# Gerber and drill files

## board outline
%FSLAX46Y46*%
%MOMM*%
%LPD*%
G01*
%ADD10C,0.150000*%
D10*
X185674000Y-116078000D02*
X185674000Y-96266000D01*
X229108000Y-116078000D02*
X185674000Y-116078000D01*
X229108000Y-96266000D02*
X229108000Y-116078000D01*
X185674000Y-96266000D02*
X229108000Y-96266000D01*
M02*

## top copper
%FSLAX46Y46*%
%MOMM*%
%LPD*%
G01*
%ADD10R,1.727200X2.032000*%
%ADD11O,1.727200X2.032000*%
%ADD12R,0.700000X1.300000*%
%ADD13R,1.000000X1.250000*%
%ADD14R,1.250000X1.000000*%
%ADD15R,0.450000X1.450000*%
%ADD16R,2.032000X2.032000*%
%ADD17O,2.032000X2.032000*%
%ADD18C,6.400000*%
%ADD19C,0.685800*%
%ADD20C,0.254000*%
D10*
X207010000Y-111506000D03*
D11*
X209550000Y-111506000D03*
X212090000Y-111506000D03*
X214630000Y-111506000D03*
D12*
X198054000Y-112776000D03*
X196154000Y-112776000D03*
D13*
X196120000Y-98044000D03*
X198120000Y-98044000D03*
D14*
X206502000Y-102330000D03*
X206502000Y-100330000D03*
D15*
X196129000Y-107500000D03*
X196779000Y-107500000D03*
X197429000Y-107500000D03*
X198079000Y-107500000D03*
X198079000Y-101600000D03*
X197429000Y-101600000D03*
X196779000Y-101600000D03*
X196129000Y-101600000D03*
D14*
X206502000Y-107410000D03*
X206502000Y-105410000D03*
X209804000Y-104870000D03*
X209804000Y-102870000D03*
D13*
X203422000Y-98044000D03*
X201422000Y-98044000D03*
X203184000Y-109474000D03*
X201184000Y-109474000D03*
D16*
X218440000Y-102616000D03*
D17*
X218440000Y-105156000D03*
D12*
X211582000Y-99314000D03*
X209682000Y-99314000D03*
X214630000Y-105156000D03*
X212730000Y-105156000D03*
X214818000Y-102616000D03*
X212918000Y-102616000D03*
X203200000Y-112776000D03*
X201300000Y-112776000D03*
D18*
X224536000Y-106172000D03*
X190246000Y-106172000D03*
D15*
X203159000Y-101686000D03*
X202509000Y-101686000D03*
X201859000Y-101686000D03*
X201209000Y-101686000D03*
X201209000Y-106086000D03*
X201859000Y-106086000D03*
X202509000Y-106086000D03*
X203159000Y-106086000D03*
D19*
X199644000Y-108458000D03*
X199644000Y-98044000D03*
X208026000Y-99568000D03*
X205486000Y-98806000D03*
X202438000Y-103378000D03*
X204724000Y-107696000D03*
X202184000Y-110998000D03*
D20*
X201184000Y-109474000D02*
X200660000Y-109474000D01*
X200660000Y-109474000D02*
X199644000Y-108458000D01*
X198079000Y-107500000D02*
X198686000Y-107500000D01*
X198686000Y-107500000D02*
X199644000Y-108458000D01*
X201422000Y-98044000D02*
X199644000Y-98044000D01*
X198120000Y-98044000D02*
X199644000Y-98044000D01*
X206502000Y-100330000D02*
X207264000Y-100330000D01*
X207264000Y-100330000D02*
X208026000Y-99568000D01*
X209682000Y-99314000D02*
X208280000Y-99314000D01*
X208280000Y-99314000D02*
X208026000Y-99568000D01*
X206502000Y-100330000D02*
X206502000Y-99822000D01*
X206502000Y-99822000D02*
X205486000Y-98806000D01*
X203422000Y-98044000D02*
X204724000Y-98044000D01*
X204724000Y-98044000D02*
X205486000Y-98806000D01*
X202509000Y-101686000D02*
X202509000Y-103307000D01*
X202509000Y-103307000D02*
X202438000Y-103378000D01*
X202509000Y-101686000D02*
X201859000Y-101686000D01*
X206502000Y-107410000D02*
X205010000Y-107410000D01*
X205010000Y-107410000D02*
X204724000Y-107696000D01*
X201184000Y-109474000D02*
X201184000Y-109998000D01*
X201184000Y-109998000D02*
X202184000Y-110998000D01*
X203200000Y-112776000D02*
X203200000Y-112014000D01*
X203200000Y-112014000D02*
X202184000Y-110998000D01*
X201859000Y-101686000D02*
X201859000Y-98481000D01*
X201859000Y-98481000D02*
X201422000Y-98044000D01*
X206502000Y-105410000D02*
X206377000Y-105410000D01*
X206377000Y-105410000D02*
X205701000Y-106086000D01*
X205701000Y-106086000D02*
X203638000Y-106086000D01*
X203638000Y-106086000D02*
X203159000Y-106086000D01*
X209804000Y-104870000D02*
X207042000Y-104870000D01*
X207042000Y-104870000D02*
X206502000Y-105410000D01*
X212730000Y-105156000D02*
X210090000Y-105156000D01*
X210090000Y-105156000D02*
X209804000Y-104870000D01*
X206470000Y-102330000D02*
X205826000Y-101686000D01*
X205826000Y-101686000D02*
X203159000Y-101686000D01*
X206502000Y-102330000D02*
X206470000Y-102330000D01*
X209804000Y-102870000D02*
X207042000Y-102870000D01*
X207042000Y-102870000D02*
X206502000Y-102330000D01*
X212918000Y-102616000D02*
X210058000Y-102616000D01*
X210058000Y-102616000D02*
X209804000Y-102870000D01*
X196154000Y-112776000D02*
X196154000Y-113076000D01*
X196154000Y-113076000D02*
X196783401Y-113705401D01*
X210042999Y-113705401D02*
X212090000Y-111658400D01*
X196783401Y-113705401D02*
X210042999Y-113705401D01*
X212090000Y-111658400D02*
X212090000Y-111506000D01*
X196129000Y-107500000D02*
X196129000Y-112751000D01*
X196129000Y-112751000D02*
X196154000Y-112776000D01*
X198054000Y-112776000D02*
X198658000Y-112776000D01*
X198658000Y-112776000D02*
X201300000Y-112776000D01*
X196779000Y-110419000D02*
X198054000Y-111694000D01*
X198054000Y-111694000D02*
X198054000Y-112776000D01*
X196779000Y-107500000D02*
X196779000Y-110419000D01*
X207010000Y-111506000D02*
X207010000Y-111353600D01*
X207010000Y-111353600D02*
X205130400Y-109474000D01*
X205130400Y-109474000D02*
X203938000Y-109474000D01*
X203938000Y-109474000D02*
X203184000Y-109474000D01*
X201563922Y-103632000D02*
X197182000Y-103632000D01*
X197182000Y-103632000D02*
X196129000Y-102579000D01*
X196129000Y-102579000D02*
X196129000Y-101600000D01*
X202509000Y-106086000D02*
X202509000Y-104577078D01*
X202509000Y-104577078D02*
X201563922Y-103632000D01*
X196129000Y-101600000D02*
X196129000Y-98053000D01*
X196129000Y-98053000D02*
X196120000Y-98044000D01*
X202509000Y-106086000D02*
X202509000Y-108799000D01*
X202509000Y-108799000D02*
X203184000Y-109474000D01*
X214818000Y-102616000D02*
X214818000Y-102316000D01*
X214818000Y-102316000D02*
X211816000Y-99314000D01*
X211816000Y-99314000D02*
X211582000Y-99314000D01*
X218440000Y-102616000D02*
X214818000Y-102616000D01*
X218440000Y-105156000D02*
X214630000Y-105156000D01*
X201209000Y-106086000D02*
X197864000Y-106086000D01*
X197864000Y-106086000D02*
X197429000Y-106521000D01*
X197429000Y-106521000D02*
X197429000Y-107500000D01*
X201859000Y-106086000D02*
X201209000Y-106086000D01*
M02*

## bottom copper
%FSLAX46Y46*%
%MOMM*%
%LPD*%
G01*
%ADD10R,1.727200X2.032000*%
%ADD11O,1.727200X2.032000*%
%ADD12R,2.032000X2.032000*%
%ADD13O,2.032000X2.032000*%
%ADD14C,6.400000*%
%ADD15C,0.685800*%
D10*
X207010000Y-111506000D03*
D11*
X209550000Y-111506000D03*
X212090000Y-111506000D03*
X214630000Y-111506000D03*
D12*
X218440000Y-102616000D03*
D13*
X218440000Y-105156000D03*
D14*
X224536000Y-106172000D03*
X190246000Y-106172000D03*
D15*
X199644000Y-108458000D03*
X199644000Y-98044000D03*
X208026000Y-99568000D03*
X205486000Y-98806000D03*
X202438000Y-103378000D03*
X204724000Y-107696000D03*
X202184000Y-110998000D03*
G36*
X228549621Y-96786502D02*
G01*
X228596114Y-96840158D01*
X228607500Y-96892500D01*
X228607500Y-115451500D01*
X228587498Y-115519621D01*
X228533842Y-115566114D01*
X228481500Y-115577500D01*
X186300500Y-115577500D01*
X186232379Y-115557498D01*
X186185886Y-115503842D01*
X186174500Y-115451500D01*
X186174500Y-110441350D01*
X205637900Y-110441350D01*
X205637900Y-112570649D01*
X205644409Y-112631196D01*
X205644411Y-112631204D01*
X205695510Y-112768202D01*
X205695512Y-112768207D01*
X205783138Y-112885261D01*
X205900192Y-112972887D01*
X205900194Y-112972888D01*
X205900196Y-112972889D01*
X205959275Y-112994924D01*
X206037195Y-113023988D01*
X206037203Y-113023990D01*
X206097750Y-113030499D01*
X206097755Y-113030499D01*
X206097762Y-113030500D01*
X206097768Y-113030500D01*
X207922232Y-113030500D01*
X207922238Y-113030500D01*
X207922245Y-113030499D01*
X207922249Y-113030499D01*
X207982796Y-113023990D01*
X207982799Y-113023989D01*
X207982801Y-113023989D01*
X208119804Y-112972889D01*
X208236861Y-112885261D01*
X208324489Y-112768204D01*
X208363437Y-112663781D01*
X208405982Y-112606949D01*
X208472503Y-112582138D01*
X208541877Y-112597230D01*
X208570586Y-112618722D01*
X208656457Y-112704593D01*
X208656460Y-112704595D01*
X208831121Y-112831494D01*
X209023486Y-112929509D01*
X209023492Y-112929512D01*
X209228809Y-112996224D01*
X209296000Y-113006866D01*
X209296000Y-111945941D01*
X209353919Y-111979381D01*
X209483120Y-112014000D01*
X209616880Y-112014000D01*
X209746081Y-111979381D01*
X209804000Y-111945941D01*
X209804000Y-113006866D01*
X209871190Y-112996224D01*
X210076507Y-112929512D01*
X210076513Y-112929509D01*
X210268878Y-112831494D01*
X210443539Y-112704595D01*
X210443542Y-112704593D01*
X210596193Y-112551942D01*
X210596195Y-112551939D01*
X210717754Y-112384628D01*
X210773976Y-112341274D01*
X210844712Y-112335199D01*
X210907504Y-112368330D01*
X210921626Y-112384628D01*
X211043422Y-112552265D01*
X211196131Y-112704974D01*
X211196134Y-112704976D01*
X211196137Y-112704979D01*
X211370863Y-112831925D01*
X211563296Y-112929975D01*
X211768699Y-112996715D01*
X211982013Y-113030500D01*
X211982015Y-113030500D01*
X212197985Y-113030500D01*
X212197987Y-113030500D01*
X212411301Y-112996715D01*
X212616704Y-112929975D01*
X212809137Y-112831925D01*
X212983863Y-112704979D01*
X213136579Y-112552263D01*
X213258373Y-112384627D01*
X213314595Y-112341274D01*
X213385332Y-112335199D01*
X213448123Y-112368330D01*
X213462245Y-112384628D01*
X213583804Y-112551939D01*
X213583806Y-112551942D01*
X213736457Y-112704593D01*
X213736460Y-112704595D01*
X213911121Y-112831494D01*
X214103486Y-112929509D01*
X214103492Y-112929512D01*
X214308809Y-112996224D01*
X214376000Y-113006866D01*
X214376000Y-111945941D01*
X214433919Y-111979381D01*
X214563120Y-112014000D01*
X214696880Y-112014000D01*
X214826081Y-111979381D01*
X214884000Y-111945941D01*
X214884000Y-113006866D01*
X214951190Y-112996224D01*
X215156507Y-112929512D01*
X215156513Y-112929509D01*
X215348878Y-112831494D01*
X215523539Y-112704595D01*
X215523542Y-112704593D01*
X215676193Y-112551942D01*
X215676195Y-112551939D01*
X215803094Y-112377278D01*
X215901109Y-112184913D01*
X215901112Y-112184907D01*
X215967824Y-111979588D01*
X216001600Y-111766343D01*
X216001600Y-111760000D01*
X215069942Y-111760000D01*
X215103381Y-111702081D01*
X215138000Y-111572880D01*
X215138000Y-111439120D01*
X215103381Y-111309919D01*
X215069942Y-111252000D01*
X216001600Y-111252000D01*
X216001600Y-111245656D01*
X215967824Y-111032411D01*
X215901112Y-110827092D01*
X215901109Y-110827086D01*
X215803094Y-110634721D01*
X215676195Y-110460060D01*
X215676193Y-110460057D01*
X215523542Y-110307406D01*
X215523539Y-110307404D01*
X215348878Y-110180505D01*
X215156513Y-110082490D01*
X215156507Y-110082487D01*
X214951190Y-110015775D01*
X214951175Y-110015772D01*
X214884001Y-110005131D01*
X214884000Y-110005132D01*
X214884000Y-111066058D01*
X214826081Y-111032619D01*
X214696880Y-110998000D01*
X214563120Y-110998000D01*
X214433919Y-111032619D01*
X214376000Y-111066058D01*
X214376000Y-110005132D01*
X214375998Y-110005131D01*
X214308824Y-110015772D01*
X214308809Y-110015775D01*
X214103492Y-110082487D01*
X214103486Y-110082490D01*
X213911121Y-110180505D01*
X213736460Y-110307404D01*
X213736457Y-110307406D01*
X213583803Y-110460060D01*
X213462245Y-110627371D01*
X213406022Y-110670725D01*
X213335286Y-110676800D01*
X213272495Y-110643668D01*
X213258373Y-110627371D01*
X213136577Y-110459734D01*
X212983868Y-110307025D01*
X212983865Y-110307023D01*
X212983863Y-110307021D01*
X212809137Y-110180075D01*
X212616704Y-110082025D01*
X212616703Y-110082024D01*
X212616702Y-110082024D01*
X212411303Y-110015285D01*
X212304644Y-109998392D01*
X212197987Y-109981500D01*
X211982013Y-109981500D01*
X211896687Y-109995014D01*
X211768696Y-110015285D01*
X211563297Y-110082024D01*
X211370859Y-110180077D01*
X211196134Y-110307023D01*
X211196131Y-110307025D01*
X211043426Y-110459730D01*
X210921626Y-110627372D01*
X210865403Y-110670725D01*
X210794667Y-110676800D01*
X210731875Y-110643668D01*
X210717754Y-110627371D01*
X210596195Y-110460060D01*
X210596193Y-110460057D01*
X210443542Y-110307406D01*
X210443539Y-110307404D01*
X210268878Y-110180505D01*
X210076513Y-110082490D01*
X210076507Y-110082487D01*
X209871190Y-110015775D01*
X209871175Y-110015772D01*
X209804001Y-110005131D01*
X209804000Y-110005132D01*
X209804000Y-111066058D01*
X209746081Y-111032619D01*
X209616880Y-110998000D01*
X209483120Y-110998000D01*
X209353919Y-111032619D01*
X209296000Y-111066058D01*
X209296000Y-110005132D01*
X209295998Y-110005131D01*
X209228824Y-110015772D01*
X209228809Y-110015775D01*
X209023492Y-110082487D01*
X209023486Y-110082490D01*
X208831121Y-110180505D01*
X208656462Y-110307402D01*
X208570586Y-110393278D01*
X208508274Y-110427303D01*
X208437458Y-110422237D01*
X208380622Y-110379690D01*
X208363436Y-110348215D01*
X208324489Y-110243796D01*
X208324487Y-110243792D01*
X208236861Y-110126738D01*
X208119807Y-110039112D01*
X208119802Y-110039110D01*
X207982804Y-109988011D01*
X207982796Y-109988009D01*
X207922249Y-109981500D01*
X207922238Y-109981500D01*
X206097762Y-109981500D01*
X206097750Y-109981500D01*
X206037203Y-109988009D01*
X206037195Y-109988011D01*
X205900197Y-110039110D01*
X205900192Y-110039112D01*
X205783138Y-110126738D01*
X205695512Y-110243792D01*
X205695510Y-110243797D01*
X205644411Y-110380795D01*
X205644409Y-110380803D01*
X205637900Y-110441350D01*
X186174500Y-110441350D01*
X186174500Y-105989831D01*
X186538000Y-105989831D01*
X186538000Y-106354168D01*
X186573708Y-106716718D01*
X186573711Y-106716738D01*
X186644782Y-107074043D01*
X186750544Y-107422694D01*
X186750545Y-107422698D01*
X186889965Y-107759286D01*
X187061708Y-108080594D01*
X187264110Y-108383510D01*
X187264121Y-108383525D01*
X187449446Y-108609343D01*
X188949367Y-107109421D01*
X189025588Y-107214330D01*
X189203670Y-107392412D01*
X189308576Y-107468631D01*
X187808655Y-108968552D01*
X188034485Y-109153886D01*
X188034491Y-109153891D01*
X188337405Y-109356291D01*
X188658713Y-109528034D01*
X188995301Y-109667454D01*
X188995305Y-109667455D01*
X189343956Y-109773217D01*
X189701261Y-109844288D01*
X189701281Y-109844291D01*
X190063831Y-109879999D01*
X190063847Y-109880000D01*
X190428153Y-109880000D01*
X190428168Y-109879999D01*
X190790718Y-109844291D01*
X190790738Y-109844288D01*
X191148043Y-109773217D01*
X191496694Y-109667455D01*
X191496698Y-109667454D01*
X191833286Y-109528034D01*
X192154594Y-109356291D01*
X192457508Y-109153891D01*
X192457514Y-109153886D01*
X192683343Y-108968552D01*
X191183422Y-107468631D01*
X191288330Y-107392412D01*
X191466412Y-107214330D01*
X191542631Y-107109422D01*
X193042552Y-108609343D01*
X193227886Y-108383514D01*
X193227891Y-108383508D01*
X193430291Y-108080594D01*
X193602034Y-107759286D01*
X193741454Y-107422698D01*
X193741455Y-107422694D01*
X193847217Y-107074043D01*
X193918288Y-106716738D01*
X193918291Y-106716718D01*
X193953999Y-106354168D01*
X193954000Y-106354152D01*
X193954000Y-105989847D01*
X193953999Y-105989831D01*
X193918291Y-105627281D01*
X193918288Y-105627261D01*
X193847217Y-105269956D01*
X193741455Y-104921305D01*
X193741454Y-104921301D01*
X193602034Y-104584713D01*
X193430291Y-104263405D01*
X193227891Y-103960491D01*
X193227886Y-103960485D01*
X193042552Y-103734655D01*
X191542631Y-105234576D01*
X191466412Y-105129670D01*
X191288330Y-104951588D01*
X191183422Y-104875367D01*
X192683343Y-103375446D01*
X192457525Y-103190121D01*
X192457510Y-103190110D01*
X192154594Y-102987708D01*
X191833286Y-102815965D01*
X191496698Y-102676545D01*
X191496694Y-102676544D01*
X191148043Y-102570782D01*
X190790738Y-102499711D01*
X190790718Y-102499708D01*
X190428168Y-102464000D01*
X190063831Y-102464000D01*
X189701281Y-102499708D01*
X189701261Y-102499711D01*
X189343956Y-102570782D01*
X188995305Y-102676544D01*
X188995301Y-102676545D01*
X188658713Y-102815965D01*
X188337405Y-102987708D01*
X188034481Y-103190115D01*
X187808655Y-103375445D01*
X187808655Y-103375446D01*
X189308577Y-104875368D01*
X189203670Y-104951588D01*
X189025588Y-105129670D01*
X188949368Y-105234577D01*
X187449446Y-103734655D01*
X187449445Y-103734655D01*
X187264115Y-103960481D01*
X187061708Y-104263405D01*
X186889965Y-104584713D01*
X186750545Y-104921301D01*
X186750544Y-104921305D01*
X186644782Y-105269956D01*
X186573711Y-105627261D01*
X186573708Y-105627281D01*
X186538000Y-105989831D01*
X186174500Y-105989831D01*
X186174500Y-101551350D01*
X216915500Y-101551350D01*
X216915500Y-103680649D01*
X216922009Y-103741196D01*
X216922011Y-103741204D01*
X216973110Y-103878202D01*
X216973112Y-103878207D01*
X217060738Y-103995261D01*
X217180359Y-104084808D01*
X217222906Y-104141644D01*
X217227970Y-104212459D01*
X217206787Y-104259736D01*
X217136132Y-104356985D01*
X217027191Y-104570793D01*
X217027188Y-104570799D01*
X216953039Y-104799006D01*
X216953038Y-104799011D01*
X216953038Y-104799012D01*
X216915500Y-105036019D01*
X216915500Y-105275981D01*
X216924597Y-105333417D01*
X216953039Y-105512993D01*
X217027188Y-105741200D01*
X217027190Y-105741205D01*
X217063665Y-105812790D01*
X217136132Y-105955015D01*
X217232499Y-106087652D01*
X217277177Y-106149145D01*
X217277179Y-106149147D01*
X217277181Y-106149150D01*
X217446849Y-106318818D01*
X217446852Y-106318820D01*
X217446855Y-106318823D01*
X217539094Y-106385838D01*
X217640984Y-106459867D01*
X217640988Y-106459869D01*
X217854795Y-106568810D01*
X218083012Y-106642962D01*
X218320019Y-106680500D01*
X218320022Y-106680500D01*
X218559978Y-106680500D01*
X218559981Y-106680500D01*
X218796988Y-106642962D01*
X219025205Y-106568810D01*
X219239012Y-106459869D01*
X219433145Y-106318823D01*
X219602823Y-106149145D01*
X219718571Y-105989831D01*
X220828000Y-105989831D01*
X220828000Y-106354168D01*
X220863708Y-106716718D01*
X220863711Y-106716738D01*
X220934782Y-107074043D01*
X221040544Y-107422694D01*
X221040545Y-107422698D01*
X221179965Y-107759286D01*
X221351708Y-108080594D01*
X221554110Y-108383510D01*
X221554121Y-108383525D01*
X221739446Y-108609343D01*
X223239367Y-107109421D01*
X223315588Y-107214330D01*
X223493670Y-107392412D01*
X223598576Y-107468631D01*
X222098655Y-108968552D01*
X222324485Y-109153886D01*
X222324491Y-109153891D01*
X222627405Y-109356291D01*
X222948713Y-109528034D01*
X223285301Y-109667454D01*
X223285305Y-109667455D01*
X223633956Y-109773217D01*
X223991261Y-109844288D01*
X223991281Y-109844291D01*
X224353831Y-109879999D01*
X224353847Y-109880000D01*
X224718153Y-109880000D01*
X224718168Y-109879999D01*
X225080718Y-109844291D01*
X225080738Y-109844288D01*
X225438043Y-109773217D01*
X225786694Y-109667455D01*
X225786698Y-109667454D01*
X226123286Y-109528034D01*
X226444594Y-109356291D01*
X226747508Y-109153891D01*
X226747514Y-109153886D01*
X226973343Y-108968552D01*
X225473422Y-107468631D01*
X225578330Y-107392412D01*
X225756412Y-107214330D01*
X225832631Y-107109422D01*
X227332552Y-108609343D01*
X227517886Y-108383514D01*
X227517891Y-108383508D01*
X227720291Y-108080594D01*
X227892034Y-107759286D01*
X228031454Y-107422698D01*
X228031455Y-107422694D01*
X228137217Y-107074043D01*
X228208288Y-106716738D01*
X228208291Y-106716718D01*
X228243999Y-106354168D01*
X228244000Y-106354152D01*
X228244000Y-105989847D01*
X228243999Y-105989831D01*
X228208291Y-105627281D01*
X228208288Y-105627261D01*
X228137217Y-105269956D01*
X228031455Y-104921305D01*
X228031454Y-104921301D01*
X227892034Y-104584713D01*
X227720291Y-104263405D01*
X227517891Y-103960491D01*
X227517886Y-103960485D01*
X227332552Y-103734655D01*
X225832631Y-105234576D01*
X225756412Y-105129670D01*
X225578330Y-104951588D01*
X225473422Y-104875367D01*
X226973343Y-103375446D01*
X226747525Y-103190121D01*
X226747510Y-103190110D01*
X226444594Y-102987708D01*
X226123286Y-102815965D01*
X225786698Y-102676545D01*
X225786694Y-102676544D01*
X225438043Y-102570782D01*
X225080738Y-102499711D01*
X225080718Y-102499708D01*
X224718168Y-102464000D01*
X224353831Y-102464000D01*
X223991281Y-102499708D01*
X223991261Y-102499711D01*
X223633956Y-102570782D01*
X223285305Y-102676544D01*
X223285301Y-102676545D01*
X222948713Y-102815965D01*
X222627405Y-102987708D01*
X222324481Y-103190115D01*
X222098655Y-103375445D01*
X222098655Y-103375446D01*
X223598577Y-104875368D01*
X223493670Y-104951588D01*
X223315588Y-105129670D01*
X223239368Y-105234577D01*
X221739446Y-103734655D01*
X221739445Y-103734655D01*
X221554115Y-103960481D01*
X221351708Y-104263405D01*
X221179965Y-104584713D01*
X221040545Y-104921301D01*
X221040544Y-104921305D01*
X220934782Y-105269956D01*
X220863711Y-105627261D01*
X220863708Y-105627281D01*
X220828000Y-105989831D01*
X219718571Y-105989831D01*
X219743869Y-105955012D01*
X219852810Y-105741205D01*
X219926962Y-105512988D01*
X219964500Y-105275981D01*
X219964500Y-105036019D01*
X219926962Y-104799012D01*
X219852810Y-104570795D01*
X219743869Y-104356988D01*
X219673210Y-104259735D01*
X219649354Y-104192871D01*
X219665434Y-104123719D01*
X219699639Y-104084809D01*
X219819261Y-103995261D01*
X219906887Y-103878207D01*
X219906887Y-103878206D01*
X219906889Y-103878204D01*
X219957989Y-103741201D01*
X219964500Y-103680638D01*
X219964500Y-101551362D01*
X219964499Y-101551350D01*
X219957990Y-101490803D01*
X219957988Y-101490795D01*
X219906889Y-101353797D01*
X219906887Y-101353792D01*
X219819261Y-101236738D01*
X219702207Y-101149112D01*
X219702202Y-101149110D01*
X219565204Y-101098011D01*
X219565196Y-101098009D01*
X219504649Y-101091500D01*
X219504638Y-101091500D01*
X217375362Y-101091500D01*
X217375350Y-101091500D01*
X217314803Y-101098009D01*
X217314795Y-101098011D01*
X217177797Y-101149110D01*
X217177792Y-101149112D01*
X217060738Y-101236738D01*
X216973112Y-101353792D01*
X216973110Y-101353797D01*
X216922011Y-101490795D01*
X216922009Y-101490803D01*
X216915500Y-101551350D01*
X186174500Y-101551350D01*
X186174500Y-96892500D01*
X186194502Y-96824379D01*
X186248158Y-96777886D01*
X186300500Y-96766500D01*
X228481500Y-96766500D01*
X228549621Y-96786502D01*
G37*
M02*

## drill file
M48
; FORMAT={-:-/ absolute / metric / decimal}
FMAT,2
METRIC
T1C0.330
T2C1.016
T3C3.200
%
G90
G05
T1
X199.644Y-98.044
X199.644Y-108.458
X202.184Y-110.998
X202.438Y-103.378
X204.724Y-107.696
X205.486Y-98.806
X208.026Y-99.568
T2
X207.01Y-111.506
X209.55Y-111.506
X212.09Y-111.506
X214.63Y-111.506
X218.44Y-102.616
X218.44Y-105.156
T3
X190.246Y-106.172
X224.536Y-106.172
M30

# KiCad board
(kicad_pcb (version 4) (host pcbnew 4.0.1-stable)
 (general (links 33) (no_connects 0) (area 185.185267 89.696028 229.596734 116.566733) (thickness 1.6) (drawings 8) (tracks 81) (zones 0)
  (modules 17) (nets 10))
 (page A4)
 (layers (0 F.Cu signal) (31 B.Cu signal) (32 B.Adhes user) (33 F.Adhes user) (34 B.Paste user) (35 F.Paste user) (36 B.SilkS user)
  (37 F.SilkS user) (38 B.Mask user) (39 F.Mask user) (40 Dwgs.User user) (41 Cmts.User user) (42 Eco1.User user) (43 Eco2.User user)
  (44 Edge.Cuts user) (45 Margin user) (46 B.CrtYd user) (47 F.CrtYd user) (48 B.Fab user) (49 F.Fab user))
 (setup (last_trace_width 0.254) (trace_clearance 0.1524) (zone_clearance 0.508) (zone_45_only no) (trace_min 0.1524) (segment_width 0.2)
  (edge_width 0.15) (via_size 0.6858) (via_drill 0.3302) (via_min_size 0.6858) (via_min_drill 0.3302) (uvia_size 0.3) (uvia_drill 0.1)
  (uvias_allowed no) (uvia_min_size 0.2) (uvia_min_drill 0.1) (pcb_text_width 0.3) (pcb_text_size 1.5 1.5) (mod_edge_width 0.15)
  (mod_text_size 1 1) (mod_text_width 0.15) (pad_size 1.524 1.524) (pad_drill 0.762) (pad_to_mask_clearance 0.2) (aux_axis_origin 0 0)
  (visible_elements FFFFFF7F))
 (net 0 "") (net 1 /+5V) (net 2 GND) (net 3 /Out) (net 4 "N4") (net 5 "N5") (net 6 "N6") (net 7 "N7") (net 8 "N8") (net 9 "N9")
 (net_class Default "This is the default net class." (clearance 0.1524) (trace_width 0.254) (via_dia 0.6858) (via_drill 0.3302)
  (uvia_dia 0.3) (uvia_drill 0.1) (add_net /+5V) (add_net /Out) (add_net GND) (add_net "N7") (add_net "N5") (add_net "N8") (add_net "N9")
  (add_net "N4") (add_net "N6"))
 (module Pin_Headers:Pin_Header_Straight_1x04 (layer F.Cu) (at 207.01 111.506 90)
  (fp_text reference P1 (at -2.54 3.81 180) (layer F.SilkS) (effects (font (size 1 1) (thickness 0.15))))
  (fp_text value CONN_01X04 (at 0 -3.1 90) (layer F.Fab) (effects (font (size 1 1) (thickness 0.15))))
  (pad 1 thru_hole rect (at 0 0 90) (size 2.032 1.7272) (drill 1.016) (layers *.Cu *.Mask F.SilkS) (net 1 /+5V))
  (pad 2 thru_hole oval (at 0 2.54 90) (size 2.032 1.7272) (drill 1.016) (layers *.Cu *.Mask F.SilkS) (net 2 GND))
  (pad 3 thru_hole oval (at 0 5.08 90) (size 2.032 1.7272) (drill 1.016) (layers *.Cu *.Mask F.SilkS) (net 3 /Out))
  (pad 4 thru_hole oval (at 0 7.62 90) (size 2.032 1.7272) (drill 1.016) (layers *.Cu *.Mask F.SilkS) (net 2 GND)))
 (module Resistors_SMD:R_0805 (layer F.Cu) (at 197.104 112.776 180)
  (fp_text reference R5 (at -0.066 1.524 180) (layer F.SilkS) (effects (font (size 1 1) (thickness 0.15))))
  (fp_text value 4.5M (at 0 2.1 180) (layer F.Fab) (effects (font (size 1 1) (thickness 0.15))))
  (pad 1 smd rect (at -0.95 0 180) (size 0.7 1.3) (layers F.Cu F.Paste F.Mask) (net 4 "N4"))
  (pad 2 smd rect (at 0.95 0 180) (size 0.7 1.3) (layers F.Cu F.Paste F.Mask) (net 3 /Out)))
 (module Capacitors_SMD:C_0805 (layer F.Cu) (at 197.12 98.044)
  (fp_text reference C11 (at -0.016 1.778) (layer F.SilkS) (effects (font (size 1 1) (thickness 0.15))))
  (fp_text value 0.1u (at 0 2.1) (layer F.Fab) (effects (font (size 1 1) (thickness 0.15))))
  (pad 1 smd rect (at -1 0) (size 1 1.25) (layers F.Cu F.Paste F.Mask) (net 1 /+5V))
  (pad 2 smd rect (at 1 0) (size 1 1.25) (layers F.Cu F.Paste F.Mask) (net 2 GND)))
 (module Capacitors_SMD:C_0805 (layer F.Cu) (at 206.502 101.33 90)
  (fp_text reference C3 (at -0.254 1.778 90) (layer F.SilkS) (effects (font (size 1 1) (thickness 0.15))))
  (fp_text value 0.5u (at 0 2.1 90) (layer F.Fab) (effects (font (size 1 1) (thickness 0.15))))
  (pad 1 smd rect (at -1 0 90) (size 1 1.25) (layers F.Cu F.Paste F.Mask) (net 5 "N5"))
  (pad 2 smd rect (at 1 0 90) (size 1 1.25) (layers F.Cu F.Paste F.Mask) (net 2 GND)))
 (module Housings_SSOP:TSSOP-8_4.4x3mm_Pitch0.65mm (layer F.Cu) (at 197.104 104.55 90)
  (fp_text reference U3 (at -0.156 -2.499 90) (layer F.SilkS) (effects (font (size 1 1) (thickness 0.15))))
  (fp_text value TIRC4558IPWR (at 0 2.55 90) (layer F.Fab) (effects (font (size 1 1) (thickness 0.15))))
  (pad 1 smd rect (at -2.95 -0.975 90) (size 1.45 0.45) (layers F.Cu F.Paste F.Mask) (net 3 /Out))
  (pad 2 smd rect (at -2.95 -0.325 90) (size 1.45 0.45) (layers F.Cu F.Paste F.Mask) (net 4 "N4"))
  (pad 3 smd rect (at -2.95 0.325 90) (size 1.45 0.45) (layers F.Cu F.Paste F.Mask) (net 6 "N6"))
  (pad 4 smd rect (at -2.95 0.975 90) (size 1.45 0.45) (layers F.Cu F.Paste F.Mask) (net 2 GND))
  (pad 5 smd rect (at 2.95 0.975 90) (size 1.45 0.45) (layers F.Cu F.Paste F.Mask))
  (pad 6 smd rect (at 2.95 0.325 90) (size 1.45 0.45) (layers F.Cu F.Paste F.Mask))
  (pad 7 smd rect (at 2.95 -0.325 90) (size 1.45 0.45) (layers F.Cu F.Paste F.Mask))
  (pad 8 smd rect (at 2.95 -0.975 90) (size 1.45 0.45) (layers F.Cu F.Paste F.Mask) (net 1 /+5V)))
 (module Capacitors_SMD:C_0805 (layer F.Cu) (at 206.502 106.41 90)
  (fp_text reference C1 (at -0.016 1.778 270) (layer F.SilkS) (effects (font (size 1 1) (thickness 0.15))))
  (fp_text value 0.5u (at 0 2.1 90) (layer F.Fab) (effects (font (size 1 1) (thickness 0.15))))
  (pad 1 smd rect (at -1 0 90) (size 1 1.25) (layers F.Cu F.Paste F.Mask) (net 2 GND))
  (pad 2 smd rect (at 1 0 90) (size 1 1.25) (layers F.Cu F.Paste F.Mask) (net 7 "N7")))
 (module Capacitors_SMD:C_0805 (layer F.Cu) (at 209.804 103.87 90)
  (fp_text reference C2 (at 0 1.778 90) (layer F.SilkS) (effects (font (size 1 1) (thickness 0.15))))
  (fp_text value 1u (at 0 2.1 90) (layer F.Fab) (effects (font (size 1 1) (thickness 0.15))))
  (pad 1 smd rect (at -1 0 90) (size 1 1.25) (layers F.Cu F.Paste F.Mask) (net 7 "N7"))
  (pad 2 smd rect (at 1 0 90) (size 1 1.25) (layers F.Cu F.Paste F.Mask) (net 5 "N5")))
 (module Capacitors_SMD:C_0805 (layer F.Cu) (at 202.422 98.044 180)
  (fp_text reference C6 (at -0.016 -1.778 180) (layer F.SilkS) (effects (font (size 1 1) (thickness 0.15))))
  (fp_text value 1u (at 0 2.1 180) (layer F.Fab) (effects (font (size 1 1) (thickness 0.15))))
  (pad 1 smd rect (at -1 0 180) (size 1 1.25) (layers F.Cu F.Paste F.Mask) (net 2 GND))
  (pad 2 smd rect (at 1 0 180) (size 1 1.25) (layers F.Cu F.Paste F.Mask) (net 2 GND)))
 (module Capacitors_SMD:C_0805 (layer F.Cu) (at 202.184 109.474 180)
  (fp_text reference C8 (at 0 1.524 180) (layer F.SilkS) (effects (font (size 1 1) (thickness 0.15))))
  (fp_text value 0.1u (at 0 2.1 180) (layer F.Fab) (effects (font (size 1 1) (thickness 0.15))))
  (pad 1 smd rect (at -1 0 180) (size 1 1.25) (layers F.Cu F.Paste F.Mask) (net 1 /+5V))
  (pad 2 smd rect (at 1 0 180) (size 1 1.25) (layers F.Cu F.Paste F.Mask) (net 2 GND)))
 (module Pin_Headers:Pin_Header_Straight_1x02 (layer F.Cu) (at 218.44 102.616)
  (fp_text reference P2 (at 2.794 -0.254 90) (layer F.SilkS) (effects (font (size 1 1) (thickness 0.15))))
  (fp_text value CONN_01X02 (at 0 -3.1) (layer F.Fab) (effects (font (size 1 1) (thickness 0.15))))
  (pad 1 thru_hole rect (at 0 0) (size 2.032 2.032) (drill 1.016) (layers *.Cu *.Mask F.SilkS) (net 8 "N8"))
  (pad 2 thru_hole oval (at 0 2.54) (size 2.032 2.032) (drill 1.016) (layers *.Cu *.Mask F.SilkS) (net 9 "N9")))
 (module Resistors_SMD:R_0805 (layer F.Cu) (at 210.632 99.314 180)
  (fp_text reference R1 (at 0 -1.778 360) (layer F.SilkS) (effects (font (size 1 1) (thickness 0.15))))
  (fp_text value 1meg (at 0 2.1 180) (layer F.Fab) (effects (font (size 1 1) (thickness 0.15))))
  (pad 1 smd rect (at -0.95 0 180) (size 0.7 1.3) (layers F.Cu F.Paste F.Mask) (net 8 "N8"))
  (pad 2 smd rect (at 0.95 0 180) (size 0.7 1.3) (layers F.Cu F.Paste F.Mask) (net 2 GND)))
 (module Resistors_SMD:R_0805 (layer F.Cu) (at 213.68 105.156 180)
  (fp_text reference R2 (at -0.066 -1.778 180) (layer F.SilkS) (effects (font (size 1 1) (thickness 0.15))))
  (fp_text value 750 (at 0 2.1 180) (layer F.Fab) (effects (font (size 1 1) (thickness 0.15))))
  (pad 1 smd rect (at -0.95 0 180) (size 0.7 1.3) (layers F.Cu F.Paste F.Mask) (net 9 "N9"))
  (pad 2 smd rect (at 0.95 0 180) (size 0.7 1.3) (layers F.Cu F.Paste F.Mask) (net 7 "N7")))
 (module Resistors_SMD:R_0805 (layer F.Cu) (at 213.868 102.616 180)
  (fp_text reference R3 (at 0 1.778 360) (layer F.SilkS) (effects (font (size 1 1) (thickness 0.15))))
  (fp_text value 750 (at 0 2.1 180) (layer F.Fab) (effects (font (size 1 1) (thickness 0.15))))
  (pad 1 smd rect (at -0.95 0 180) (size 0.7 1.3) (layers F.Cu F.Paste F.Mask) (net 8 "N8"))
  (pad 2 smd rect (at 0.95 0 180) (size 0.7 1.3) (layers F.Cu F.Paste F.Mask) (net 5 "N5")))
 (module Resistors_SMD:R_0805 (layer F.Cu) (at 202.25 112.776 180)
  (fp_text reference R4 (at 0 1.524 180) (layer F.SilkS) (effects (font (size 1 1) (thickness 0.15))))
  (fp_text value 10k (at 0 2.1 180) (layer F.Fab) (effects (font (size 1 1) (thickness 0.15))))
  (pad 1 smd rect (at -0.95 0 180) (size 0.7 1.3) (layers F.Cu F.Paste F.Mask) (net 2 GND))
  (pad 2 smd rect (at 0.95 0 180) (size 0.7 1.3) (layers F.Cu F.Paste F.Mask) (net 4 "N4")))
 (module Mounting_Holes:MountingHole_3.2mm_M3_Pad (layer F.Cu) (at 224.536 106.172)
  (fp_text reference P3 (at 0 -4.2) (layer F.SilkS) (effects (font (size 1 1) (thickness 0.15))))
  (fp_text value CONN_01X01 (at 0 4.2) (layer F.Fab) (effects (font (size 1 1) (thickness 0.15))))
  (pad 1 thru_hole circle (at 0 0) (size 6.4 6.4) (drill 3.2) (layers *.Cu *.Mask F.SilkS) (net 2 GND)))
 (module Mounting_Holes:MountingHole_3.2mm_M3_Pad (layer F.Cu) (at 190.246 106.172)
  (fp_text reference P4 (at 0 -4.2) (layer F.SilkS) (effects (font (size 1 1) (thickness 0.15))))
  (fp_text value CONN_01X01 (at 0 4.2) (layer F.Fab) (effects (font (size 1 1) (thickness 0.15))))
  (pad 1 thru_hole circle (at 0 0) (size 6.4 6.4) (drill 3.2) (layers *.Cu *.Mask F.SilkS) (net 2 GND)))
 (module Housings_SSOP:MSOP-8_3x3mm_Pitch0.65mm (layer F.Cu) (at 202.184 103.886 270)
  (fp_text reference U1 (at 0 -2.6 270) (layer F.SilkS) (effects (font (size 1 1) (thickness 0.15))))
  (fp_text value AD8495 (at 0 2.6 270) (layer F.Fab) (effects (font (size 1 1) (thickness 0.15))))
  (pad 1 smd rect (at -2.2 -0.975 270) (size 1.45 0.45) (layers F.Cu F.Paste F.Mask) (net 5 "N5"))
  (pad 2 smd rect (at -2.2 -0.325 270) (size 1.45 0.45) (layers F.Cu F.Paste F.Mask) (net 2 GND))
  (pad 3 smd rect (at -2.2 0.325 270) (size 1.45 0.45) (layers F.Cu F.Paste F.Mask) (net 2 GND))
  (pad 4 smd rect (at -2.2 0.975 270) (size 1.45 0.45) (layers F.Cu F.Paste F.Mask))
  (pad 5 smd rect (at 2.2 0.975 270) (size 1.45 0.45) (layers F.Cu F.Paste F.Mask) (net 6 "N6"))
  (pad 6 smd rect (at 2.2 0.325 270) (size 1.45 0.45) (layers F.Cu F.Paste F.Mask) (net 6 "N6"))
  (pad 7 smd rect (at 2.2 -0.325 270) (size 1.45 0.45) (layers F.Cu F.Paste F.Mask) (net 1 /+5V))
  (pad 8 smd rect (at 2.2 -0.975 270) (size 1.45 0.45) (layers F.Cu F.Paste F.Mask) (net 7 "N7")))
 (gr_line (start 185.674 116.078) (end 185.674 96.266) (layer Edge.Cuts) (width 0.15))
 (gr_line (start 229.108 116.078) (end 185.674 116.078) (layer Edge.Cuts) (width 0.15))
 (gr_line (start 229.108 96.266) (end 229.108 116.078) (layer Edge.Cuts) (width 0.15))
 (gr_line (start 185.674 96.266) (end 229.108 96.266) (layer Edge.Cuts) (width 0.15))
 (segment (start 201.184 109.474) (end 200.66 109.474) (width 0.254) (layer F.Cu) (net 2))
 (segment (start 200.66 109.474) (end 199.644 108.458) (width 0.254) (layer F.Cu) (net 2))
 (segment (start 198.079 107.5) (end 198.686 107.5) (width 0.254) (layer F.Cu) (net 2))
 (segment (start 198.686 107.5) (end 199.644 108.458) (width 0.254) (layer F.Cu) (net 2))
 (via (at 199.644 108.458) (size 0.6858) (drill 0.3302) (layers F.Cu B.Cu) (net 2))
 (segment (start 201.422 98.044) (end 199.644 98.044) (width 0.254) (layer F.Cu) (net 2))
 (segment (start 198.12 98.044) (end 199.644 98.044) (width 0.254) (layer F.Cu) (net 2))
 (via (at 199.644 98.044) (size 0.6858) (drill 0.3302) (layers F.Cu B.Cu) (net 2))
 (segment (start 206.502 100.33) (end 207.264 100.33) (width 0.254) (layer F.Cu) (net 2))
 (segment (start 207.264 100.33) (end 208.026 99.568) (width 0.254) (layer F.Cu) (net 2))
 (segment (start 209.682 99.314) (end 208.28 99.314) (width 0.254) (layer F.Cu) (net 2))
 (segment (start 208.28 99.314) (end 208.026 99.568) (width 0.254) (layer F.Cu) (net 2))
 (via (at 208.026 99.568) (size 0.6858) (drill 0.3302) (layers F.Cu B.Cu) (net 2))
 (segment (start 206.502 100.33) (end 206.502 99.822) (width 0.254) (layer F.Cu) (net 2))
 (segment (start 206.502 99.822) (end 205.486 98.806) (width 0.254) (layer F.Cu) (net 2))
 (segment (start 203.422 98.044) (end 204.724 98.044) (width 0.254) (layer F.Cu) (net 2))
 (segment (start 204.724 98.044) (end 205.486 98.806) (width 0.254) (layer F.Cu) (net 2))
 (via (at 205.486 98.806) (size 0.6858) (drill 0.3302) (layers F.Cu B.Cu) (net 2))
 (segment (start 202.509 101.686) (end 202.509 103.307) (width 0.254) (layer F.Cu) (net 2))
 (segment (start 202.509 103.307) (end 202.438 103.378) (width 0.254) (layer F.Cu) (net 2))
 (via (at 202.438 103.378) (size 0.6858) (drill 0.3302) (layers F.Cu B.Cu) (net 2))
 (segment (start 202.509 101.686) (end 201.859 101.686) (width 0.254) (layer F.Cu) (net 2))
 (segment (start 206.502 107.41) (end 205.01 107.41) (width 0.254) (layer F.Cu) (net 2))
 (via (at 204.724 107.696) (size 0.6858) (drill 0.3302) (layers F.Cu B.Cu) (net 2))
 (segment (start 205.01 107.41) (end 204.724 107.696) (width 0.254) (layer F.Cu) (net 2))
 (segment (start 201.184 109.474) (end 201.184 109.998) (width 0.254) (layer F.Cu) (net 2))
 (segment (start 201.184 109.998) (end 202.184 110.998) (width 0.254) (layer F.Cu) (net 2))
 (segment (start 203.2 112.776) (end 203.2 112.014) (width 0.254) (layer F.Cu) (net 2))
 (via (at 202.184 110.998) (size 0.6858) (drill 0.3302) (layers F.Cu B.Cu) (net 2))
 (segment (start 203.2 112.014) (end 202.184 110.998) (width 0.254) (layer F.Cu) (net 2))
 (segment (start 201.859 101.686) (end 201.859 98.481) (width 0.254) (layer F.Cu) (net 2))
 (segment (start 201.859 98.481) (end 201.422 98.044) (width 0.254) (layer F.Cu) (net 2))
 (segment (start 206.502 105.41) (end 206.377 105.41) (width 0.254) (layer F.Cu) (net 7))
 (segment (start 206.377 105.41) (end 205.701 106.086) (width 0.254) (layer F.Cu) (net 7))
 (segment (start 205.701 106.086) (end 203.638 106.086) (width 0.254) (layer F.Cu) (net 7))
 (segment (start 203.638 106.086) (end 203.159 106.086) (width 0.254) (layer F.Cu) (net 7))
 (segment (start 209.804 104.87) (end 207.042 104.87) (width 0.254) (layer F.Cu) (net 7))
 (segment (start 207.042 104.87) (end 206.502 105.41) (width 0.254) (layer F.Cu) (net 7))
 (segment (start 212.73 105.156) (end 210.09 105.156) (width 0.254) (layer F.Cu) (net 7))
 (segment (start 210.09 105.156) (end 209.804 104.87) (width 0.254) (layer F.Cu) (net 7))
 (segment (start 206.47 102.33) (end 205.826 101.686) (width 0.254) (layer F.Cu) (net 5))
 (segment (start 205.826 101.686) (end 203.159 101.686) (width 0.254) (layer F.Cu) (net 5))
 (segment (start 206.502 102.33) (end 206.47 102.33) (width 0.254) (layer F.Cu) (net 5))
 (segment (start 209.804 102.87) (end 207.042 102.87) (width 0.254) (layer F.Cu) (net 5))
 (segment (start 207.042 102.87) (end 206.502 102.33) (width 0.254) (layer F.Cu) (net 5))
 (segment (start 212.918 102.616) (end 210.058 102.616) (width 0.254) (layer F.Cu) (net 5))
 (segment (start 210.058 102.616) (end 209.804 102.87) (width 0.254) (layer F.Cu) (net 5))
 (segment (start 196.154 112.776) (end 196.154 113.076) (width 0.254) (layer F.Cu) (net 3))
 (segment (start 196.154 113.076) (end 196.783401 113.705401) (width 0.254) (layer F.Cu) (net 3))
 (segment (start 210.042999 113.705401) (end 212.09 111.6584) (width 0.254) (layer F.Cu) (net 3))
 (segment (start 196.783401 113.705401) (end 210.042999 113.705401) (width 0.254) (layer F.Cu) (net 3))
 (segment (start 212.09 111.6584) (end 212.09 111.506) (width 0.254) (layer F.Cu) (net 3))
 (segment (start 196.129 107.5) (end 196.129 112.751) (width 0.254) (layer F.Cu) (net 3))
 (segment (start 196.129 112.751) (end 196.154 112.776) (width 0.254) (layer F.Cu) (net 3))
 (segment (start 198.054 112.776) (end 198.658 112.776) (width 0.254) (layer F.Cu) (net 4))
 (segment (start 198.658 112.776) (end 201.3 112.776) (width 0.254) (layer F.Cu) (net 4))
 (segment (start 196.779 110.419) (end 198.054 111.694) (width 0.254) (layer F.Cu) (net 4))
 (segment (start 198.054 111.694) (end 198.054 112.776) (width 0.254) (layer F.Cu) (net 4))
 (segment (start 196.779 107.5) (end 196.779 110.419) (width 0.254) (layer F.Cu) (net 4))
 (segment (start 207.01 111.506) (end 207.01 111.3536) (width 0.254) (layer F.Cu) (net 1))
 (segment (start 207.01 111.3536) (end 205.1304 109.474) (width 0.254) (layer F.Cu) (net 1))
 (segment (start 205.1304 109.474) (end 203.938 109.474) (width 0.254) (layer F.Cu) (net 1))
 (segment (start 203.938 109.474) (end 203.184 109.474) (width 0.254) (layer F.Cu) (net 1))
 (segment (start 201.563922 103.632) (end 197.182 103.632) (width 0.254) (layer F.Cu) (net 1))
 (segment (start 197.182 103.632) (end 196.129 102.579) (width 0.254) (layer F.Cu) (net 1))
 (segment (start 196.129 102.579) (end 196.129 101.6) (width 0.254) (layer F.Cu) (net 1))
 (segment (start 202.509 106.086) (end 202.509 104.577078) (width 0.254) (layer F.Cu) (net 1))
 (segment (start 202.509 104.577078) (end 201.563922 103.632) (width 0.254) (layer F.Cu) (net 1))
 (segment (start 196.129 101.6) (end 196.129 98.053) (width 0.254) (layer F.Cu) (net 1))
 (segment (start 196.129 98.053) (end 196.12 98.044) (width 0.254) (layer F.Cu) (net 1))
 (segment (start 202.509 106.086) (end 202.509 108.799) (width 0.254) (layer F.Cu) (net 1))
 (segment (start 202.509 108.799) (end 203.184 109.474) (width 0.254) (layer F.Cu) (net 1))
 (segment (start 214.818 102.616) (end 214.818 102.316) (width 0.254) (layer F.Cu) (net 8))
 (segment (start 214.818 102.316) (end 211.816 99.314) (width 0.254) (layer F.Cu) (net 8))
 (segment (start 211.816 99.314) (end 211.582 99.314) (width 0.254) (layer F.Cu) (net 8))
 (segment (start 218.44 102.616) (end 214.818 102.616) (width 0.254) (layer F.Cu) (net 8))
 (segment (start 218.44 105.156) (end 214.63 105.156) (width 0.254) (layer F.Cu) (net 9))
 (segment (start 201.209 106.086) (end 197.864 106.086) (width 0.254) (layer F.Cu) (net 6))
 (segment (start 197.864 106.086) (end 197.429 106.521) (width 0.254) (layer F.Cu) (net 6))
 (segment (start 197.429 106.521) (end 197.429 107.5) (width 0.254) (layer F.Cu) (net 6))
 (segment (start 201.859 106.086) (end 201.209 106.086) (width 0.254) (layer F.Cu) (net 6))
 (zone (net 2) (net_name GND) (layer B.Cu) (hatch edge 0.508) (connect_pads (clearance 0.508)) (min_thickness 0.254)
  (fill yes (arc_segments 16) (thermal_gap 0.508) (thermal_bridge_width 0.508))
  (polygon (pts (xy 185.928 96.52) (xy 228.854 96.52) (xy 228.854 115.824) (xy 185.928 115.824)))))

